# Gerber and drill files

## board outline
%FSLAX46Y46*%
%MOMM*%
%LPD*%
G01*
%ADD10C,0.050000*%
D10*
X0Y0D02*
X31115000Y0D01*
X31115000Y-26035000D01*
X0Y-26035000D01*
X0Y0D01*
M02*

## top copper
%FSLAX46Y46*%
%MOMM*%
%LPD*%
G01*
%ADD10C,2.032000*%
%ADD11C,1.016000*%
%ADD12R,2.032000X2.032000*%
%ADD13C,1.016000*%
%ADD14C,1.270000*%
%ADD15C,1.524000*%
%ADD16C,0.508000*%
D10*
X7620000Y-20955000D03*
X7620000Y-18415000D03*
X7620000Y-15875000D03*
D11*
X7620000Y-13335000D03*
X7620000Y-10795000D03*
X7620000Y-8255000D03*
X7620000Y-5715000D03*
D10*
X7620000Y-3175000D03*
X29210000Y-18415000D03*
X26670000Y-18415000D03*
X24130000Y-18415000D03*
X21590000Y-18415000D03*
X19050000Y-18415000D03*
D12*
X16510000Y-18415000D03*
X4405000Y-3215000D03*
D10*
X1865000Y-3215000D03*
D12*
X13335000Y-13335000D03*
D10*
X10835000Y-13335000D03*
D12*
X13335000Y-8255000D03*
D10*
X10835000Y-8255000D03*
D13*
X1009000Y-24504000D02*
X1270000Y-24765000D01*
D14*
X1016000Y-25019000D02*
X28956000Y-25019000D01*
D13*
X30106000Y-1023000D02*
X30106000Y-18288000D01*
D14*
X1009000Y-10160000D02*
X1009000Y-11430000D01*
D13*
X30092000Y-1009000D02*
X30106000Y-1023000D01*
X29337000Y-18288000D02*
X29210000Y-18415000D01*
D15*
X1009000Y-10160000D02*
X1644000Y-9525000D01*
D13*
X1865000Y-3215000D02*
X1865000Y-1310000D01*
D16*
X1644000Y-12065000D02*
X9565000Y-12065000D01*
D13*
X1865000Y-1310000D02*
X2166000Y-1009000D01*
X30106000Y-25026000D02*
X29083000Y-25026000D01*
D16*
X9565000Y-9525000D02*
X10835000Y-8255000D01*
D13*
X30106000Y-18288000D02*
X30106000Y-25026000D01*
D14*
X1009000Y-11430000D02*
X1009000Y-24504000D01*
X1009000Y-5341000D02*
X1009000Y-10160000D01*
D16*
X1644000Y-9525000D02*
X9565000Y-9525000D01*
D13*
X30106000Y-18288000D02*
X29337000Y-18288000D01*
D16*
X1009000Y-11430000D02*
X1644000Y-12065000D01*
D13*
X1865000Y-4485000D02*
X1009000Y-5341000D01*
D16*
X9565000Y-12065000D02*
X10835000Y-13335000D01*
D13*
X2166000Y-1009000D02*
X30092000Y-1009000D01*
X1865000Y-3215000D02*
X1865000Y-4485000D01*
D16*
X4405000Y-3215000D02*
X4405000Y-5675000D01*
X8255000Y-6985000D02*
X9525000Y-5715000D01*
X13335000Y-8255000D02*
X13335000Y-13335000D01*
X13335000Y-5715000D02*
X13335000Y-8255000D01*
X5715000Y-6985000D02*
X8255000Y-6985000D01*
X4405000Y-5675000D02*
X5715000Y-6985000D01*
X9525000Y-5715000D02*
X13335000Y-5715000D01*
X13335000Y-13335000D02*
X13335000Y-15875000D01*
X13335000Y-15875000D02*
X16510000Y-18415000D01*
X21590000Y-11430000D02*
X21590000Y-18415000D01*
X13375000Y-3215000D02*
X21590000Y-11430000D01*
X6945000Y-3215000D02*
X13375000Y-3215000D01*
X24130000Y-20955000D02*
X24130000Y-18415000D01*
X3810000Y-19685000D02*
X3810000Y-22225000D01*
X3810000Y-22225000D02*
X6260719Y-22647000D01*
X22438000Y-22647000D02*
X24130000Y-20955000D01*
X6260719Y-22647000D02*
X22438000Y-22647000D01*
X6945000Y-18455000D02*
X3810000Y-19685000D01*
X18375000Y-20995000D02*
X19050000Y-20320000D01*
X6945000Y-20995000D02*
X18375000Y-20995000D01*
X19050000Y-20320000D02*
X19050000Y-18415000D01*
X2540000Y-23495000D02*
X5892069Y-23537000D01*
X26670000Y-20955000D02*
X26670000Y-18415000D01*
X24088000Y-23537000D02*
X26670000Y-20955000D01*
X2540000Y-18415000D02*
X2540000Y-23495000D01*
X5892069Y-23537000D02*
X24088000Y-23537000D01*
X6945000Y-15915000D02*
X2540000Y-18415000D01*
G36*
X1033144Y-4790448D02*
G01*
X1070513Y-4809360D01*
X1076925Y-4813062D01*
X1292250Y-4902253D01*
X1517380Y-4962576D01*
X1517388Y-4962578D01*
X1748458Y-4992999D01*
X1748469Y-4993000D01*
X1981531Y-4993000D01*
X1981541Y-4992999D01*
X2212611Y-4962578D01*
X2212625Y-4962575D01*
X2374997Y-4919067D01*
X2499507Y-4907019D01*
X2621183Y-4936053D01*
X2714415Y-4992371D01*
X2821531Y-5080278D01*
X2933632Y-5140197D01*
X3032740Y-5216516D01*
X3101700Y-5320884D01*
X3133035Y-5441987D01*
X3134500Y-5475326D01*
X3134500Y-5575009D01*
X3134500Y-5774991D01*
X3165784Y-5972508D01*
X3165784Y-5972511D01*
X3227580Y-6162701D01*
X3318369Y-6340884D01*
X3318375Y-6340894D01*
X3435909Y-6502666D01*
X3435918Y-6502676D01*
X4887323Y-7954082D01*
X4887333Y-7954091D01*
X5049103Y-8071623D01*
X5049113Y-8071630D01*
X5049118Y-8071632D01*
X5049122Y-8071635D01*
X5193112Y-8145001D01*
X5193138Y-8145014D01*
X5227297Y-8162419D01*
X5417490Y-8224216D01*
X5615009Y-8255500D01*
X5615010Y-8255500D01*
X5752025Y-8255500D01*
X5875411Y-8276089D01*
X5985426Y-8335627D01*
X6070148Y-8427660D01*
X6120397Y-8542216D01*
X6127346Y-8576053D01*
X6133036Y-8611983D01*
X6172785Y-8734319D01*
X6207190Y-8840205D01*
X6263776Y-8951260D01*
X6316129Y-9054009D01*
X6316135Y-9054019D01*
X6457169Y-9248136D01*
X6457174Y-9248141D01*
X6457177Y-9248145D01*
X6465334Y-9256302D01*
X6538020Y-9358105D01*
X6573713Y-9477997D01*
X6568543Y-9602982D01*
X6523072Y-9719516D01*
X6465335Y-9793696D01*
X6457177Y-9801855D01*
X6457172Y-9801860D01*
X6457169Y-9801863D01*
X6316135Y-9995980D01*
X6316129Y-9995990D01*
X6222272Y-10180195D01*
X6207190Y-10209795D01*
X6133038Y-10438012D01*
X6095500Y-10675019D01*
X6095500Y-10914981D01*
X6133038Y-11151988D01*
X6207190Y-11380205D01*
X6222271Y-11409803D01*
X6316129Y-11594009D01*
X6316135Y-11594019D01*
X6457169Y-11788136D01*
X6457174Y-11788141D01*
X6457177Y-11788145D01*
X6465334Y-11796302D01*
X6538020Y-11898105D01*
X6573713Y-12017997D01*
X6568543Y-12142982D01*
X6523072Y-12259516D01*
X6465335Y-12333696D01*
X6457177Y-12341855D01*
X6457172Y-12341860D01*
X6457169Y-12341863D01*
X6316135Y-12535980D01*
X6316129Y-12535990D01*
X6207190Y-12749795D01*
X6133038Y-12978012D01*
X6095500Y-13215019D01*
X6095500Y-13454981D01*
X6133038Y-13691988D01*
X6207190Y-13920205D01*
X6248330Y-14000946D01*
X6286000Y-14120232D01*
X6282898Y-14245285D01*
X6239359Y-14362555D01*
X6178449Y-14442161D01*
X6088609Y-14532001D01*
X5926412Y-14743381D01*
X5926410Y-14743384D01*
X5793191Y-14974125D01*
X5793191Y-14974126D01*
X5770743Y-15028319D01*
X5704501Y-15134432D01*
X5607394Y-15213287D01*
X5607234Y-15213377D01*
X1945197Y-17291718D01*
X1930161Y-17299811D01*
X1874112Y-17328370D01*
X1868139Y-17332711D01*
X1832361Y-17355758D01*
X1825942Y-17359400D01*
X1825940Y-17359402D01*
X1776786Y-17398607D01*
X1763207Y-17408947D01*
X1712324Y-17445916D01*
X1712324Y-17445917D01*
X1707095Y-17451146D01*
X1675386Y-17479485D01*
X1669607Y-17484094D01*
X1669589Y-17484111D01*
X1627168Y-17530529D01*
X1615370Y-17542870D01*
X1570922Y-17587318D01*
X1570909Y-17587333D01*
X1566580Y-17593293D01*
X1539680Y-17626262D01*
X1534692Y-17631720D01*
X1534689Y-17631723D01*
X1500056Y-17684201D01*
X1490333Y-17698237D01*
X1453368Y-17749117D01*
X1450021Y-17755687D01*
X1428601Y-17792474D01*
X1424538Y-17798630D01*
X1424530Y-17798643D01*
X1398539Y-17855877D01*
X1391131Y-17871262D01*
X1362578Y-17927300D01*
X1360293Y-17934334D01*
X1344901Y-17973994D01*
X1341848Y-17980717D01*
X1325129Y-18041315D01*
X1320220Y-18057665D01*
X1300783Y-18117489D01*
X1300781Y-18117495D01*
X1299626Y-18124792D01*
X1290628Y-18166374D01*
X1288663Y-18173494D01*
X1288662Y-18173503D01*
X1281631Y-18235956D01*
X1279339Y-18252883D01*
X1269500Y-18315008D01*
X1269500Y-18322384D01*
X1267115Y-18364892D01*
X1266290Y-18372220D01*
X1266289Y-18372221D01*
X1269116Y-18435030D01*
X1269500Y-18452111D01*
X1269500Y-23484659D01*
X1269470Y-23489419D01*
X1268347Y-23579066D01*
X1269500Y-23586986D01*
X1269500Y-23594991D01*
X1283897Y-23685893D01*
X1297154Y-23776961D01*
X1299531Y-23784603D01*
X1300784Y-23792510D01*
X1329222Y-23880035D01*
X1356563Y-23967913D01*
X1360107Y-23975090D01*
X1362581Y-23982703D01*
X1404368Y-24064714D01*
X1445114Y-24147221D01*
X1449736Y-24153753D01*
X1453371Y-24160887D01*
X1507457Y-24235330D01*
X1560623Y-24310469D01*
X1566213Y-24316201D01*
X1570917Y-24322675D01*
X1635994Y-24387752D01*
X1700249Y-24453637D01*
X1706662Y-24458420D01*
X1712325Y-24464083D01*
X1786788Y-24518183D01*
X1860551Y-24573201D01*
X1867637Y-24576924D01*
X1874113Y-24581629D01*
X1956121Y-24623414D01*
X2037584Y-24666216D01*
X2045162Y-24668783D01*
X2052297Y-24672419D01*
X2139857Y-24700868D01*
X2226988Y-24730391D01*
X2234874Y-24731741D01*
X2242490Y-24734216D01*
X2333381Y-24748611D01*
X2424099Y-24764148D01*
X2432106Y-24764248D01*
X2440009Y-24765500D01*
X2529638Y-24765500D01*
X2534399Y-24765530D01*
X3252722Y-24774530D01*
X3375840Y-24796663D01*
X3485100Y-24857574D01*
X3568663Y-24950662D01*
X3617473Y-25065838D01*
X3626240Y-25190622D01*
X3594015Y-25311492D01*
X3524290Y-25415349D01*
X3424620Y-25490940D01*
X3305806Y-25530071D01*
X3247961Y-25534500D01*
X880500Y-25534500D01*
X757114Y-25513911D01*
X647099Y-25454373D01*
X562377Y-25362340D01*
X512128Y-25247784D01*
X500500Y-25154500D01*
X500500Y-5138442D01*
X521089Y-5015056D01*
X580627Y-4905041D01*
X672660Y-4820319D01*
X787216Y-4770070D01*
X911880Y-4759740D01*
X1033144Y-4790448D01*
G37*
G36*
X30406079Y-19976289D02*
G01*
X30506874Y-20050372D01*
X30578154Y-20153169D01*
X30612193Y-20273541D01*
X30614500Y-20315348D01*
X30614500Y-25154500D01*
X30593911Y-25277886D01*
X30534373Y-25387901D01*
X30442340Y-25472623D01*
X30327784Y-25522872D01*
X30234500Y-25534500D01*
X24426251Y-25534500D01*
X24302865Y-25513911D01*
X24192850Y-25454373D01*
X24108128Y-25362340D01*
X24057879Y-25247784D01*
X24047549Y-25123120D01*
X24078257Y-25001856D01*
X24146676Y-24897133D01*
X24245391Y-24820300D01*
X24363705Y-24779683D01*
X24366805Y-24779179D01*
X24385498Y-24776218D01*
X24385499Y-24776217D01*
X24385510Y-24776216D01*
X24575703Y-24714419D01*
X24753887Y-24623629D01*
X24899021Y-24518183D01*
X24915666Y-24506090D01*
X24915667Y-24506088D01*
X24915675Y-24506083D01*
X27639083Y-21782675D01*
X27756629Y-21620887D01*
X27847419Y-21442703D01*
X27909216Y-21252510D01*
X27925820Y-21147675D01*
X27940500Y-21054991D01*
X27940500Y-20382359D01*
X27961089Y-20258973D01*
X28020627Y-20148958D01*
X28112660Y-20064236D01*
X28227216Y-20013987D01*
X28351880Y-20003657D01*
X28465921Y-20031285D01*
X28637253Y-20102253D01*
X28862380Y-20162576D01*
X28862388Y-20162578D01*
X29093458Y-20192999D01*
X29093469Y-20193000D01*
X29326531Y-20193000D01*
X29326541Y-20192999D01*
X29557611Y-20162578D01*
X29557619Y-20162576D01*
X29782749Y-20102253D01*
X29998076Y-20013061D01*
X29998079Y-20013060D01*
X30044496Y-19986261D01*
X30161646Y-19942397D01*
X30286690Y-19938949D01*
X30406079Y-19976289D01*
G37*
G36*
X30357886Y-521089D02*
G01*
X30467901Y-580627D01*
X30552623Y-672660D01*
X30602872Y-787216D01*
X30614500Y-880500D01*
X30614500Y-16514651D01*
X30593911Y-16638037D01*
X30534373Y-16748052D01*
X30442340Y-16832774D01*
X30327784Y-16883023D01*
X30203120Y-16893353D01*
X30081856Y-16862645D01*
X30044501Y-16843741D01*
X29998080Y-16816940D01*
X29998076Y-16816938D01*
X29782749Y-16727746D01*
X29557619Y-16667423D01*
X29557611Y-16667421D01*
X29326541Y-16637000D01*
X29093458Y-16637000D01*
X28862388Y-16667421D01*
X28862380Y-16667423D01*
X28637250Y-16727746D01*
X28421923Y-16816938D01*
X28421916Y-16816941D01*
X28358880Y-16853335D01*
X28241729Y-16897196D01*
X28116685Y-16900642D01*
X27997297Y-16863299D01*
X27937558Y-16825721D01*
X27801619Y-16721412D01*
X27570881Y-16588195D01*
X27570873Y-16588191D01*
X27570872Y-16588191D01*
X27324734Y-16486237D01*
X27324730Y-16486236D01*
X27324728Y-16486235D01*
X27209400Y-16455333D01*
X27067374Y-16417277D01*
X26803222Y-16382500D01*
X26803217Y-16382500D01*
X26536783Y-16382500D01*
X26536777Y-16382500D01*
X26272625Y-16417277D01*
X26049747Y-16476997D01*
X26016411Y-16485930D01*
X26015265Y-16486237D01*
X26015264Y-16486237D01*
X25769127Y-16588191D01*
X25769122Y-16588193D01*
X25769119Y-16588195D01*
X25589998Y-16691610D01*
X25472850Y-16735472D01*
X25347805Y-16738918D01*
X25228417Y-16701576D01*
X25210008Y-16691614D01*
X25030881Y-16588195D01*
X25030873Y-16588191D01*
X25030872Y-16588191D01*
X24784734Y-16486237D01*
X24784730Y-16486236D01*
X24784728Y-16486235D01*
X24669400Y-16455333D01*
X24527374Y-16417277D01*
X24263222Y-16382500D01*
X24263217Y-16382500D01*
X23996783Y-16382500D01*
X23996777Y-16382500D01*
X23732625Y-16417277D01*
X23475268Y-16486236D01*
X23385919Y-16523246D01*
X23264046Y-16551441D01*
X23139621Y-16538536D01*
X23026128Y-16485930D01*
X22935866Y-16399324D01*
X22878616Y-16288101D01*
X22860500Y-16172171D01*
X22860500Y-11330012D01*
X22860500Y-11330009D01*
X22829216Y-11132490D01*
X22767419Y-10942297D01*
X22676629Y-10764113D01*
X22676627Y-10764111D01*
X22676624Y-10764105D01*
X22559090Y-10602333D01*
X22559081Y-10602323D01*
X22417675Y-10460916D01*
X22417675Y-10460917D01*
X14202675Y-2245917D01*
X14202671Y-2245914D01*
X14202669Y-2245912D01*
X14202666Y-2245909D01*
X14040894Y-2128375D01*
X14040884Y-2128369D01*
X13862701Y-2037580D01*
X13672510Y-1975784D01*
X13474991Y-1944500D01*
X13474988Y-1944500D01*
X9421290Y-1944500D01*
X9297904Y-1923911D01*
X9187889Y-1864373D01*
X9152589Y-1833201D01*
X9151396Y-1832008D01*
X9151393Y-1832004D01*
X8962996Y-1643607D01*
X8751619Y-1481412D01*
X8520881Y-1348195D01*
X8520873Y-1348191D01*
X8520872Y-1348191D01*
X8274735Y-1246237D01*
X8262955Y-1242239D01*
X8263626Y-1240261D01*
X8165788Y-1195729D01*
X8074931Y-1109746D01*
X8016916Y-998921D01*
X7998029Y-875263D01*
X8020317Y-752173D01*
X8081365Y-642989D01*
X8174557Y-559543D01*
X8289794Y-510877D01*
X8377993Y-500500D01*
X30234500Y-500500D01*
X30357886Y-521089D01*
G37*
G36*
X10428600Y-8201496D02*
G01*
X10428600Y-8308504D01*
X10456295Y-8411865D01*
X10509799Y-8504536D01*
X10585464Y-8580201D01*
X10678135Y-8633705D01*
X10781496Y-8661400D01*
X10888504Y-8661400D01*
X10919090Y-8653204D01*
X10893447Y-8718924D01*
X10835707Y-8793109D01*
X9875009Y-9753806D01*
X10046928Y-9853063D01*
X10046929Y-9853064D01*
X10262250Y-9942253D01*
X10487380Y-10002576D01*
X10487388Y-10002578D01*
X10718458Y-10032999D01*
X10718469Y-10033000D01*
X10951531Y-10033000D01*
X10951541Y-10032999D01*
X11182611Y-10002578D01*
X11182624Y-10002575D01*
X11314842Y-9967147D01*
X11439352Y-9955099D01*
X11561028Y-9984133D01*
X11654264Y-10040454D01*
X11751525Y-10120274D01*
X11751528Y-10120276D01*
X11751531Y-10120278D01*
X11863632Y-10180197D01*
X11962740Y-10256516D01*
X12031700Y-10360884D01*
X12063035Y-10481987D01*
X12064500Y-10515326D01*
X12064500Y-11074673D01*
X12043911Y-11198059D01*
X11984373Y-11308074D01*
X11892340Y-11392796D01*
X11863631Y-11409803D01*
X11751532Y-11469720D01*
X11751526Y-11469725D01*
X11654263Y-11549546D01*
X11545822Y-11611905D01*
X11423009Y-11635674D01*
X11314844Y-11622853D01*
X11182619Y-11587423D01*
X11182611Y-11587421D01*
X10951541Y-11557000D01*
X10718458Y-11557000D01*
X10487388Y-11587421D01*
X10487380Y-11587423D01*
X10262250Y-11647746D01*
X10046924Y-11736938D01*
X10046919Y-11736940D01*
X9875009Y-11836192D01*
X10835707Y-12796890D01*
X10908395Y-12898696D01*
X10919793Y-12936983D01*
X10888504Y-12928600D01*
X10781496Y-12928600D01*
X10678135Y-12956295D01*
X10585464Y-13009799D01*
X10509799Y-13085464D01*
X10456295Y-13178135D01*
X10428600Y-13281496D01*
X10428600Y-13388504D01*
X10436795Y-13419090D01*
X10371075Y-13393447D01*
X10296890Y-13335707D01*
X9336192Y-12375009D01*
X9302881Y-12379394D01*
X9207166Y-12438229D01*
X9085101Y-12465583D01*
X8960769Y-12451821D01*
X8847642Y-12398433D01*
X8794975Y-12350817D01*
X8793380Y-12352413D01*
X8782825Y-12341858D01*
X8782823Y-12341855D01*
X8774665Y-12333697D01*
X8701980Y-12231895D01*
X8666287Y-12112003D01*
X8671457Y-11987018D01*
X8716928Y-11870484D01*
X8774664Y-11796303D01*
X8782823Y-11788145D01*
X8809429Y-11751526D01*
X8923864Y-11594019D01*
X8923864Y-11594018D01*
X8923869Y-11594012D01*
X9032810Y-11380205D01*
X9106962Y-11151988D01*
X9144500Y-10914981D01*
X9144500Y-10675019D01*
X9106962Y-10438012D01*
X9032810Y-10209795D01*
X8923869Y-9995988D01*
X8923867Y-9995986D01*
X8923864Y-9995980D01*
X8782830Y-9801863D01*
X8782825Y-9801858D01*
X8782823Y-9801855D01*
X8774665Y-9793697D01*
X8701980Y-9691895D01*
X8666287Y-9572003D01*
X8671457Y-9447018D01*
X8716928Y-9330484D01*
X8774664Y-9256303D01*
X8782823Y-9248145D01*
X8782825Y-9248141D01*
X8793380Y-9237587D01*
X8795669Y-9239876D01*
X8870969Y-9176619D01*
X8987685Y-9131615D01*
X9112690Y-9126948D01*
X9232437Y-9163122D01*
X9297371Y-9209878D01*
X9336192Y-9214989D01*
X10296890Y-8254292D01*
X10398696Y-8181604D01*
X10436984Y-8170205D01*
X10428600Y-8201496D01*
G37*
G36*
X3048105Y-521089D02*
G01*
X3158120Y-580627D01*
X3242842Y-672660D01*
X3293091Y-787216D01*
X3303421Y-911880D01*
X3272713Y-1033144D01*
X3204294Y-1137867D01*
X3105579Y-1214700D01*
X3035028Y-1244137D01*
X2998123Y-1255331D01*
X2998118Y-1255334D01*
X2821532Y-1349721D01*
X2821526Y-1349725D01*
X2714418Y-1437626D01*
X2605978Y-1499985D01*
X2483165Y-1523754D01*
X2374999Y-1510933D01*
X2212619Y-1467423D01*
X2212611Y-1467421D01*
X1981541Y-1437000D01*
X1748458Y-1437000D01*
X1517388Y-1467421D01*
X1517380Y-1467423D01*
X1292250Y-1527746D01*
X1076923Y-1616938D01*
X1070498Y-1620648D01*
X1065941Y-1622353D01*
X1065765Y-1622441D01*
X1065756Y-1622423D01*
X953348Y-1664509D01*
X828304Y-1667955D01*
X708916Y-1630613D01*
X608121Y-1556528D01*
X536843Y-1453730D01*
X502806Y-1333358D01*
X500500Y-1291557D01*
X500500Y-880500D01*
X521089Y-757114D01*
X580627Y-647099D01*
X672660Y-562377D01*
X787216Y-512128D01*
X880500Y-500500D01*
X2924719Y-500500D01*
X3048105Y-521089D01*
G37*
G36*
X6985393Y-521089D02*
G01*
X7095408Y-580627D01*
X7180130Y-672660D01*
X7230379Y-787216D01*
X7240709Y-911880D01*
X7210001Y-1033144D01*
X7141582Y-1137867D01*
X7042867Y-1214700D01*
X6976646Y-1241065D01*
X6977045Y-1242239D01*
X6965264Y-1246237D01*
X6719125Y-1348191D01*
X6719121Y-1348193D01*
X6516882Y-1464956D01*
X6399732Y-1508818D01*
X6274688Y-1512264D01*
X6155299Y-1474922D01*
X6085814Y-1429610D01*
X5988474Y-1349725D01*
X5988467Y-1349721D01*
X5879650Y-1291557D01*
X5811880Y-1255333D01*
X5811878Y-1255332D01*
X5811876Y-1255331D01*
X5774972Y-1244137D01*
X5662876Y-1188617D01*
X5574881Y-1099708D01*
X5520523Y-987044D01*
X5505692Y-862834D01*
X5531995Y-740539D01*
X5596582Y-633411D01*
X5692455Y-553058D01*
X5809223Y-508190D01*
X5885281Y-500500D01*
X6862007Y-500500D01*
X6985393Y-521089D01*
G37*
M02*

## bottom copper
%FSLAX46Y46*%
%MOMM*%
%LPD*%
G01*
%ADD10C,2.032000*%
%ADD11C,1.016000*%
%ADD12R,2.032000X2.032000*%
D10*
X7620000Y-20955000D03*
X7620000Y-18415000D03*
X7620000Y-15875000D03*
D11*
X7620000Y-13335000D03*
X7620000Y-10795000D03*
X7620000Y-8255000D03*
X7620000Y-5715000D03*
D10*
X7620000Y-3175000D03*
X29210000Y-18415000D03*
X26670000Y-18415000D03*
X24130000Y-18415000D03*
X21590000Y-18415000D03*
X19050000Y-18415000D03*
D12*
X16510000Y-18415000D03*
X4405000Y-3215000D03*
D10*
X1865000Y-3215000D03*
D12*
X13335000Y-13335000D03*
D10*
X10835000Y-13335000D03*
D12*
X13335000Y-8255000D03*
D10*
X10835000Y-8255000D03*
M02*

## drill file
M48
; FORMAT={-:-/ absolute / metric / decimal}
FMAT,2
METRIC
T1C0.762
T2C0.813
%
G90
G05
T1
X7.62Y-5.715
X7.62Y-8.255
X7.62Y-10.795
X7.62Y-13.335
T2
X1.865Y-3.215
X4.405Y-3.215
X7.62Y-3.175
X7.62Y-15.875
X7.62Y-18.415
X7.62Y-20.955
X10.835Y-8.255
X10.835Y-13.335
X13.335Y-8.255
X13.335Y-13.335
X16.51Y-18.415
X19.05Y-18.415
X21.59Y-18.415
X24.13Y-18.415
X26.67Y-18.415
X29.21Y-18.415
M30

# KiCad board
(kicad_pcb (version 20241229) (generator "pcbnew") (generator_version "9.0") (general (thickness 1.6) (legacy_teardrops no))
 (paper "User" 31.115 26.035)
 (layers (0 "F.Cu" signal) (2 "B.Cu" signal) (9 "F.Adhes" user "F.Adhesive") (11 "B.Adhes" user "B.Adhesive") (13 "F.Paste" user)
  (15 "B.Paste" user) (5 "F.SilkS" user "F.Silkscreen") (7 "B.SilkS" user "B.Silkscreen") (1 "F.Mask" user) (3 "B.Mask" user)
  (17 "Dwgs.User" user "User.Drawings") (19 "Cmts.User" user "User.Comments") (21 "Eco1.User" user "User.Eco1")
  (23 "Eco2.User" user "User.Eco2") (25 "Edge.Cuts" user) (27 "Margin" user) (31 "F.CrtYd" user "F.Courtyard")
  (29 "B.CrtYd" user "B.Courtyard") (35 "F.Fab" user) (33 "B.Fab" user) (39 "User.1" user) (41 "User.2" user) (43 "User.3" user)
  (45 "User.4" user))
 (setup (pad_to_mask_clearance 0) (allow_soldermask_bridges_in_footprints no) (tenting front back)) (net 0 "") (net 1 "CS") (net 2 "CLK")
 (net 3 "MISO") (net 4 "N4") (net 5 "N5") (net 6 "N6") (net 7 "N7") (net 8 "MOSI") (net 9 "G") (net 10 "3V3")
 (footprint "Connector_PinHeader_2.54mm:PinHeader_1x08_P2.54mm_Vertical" (layer "F.Cu") (at 7.62 20.955 180)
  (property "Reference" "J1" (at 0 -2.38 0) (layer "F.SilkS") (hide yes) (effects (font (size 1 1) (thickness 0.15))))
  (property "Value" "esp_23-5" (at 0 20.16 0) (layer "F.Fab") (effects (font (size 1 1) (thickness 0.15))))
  (pad "1" thru_hole circle (at 0 0 180) (size 2.032 2.032) (drill 0.8128) (layers "*.Cu" "*.Mask") (remove_unused_layers no) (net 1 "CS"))
  (pad "2" thru_hole circle (at 0 2.54 180) (size 2.032 2.032) (drill 0.8128) (layers "*.Cu" "*.Mask") (remove_unused_layers no)
   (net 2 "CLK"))
  (pad "3" thru_hole circle (at 0 5.08 180) (size 2.032 2.032) (drill 0.8128) (layers "*.Cu" "*.Mask") (remove_unused_layers no)
   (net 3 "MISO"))
  (pad "4" thru_hole circle (at 0 7.62 180) (size 1.016 1.016) (drill 0.762) (layers "*.Cu" "*.Mask") (remove_unused_layers no) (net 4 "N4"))
  (pad "5" thru_hole circle (at 0 10.16 180) (size 1.016 1.016) (drill 0.762) (layers "*.Cu" "*.Mask") (remove_unused_layers no)
   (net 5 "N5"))
  (pad "6" thru_hole circle (at 0 12.7 180) (size 1.016 1.016) (drill 0.762) (layers "*.Cu" "*.Mask") (remove_unused_layers no) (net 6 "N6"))
  (pad "7" thru_hole circle (at 0 15.24 180) (size 1.016 1.016) (drill 0.762) (layers "*.Cu" "*.Mask") (remove_unused_layers no)
   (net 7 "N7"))
  (pad "8" thru_hole circle (at 0 17.78 180) (size 2.032 2.032) (drill 0.8128) (layers "*.Cu" "*.Mask") (remove_unused_layers no)
   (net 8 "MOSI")))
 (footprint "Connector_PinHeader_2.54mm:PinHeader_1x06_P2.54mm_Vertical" (layer "F.Cu") (at 29.21 18.415 -90)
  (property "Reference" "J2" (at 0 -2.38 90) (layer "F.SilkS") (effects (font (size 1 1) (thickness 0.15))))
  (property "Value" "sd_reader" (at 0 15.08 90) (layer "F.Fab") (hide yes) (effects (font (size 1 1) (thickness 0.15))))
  (pad "1" thru_hole circle (at 0 0 270) (size 2.032 2.032) (drill 0.8128) (layers "*.Cu" "*.Mask") (remove_unused_layers no) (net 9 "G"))
  (pad "2" thru_hole circle (at 0 2.54 270) (size 2.032 2.032) (drill 0.8128) (layers "*.Cu" "*.Mask") (remove_unused_layers no)
   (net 3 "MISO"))
  (pad "3" thru_hole circle (at 0 5.08 270) (size 2.032 2.032) (drill 0.8128) (layers "*.Cu" "*.Mask") (remove_unused_layers no)
   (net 2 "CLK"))
  (pad "4" thru_hole circle (at 0 7.62 270) (size 2.032 2.032) (drill 0.8128) (layers "*.Cu" "*.Mask") (remove_unused_layers no)
   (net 8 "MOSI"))
  (pad "5" thru_hole circle (at 0 10.16 270) (size 2.032 2.032) (drill 0.8128) (layers "*.Cu" "*.Mask") (remove_unused_layers no)
   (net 1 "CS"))
  (pad "6" thru_hole rect (at 0 12.7 270) (size 2.032 2.032) (drill 0.8128) (layers "*.Cu" "*.Mask") (remove_unused_layers no)
   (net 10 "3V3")))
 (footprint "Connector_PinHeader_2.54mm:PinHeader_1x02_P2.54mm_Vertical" (layer "F.Cu") (at 4.405 3.215 -90)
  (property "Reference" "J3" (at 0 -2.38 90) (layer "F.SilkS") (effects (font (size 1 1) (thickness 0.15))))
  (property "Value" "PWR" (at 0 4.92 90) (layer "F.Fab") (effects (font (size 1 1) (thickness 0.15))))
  (pad "1" thru_hole rect (at 0 0 270) (size 2.032 2.032) (drill 0.8128) (layers "*.Cu" "*.Mask") (remove_unused_layers no) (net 10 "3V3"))
  (pad "2" thru_hole circle (at 0 2.54 270) (size 2.032 2.032) (drill 0.8128) (layers "*.Cu" "*.Mask") (remove_unused_layers no) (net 9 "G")))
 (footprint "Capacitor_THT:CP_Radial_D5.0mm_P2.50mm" (layer "F.Cu") (at 13.335 13.335 180)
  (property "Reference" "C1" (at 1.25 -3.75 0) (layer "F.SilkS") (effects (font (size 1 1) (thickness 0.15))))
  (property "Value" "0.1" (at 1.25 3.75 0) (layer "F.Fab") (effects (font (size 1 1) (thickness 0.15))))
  (pad "1" thru_hole rect (at 0 0 180) (size 2.032 2.032) (drill 0.8128) (layers "*.Cu" "*.Mask") (remove_unused_layers no) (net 10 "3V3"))
  (pad "2" thru_hole circle (at 2.5 0 180) (size 2.032 2.032) (drill 0.8128) (layers "*.Cu" "*.Mask") (remove_unused_layers no) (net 9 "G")))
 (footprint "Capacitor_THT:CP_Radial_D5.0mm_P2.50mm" (layer "F.Cu") (at 13.335 8.255 180)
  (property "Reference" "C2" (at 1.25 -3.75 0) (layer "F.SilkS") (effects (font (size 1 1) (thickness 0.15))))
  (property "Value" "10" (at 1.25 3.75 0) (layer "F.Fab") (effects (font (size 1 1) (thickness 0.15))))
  (pad "1" thru_hole rect (at 0 0 180) (size 2.032 2.032) (drill 0.8128) (layers "*.Cu" "*.Mask") (remove_unused_layers no) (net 10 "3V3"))
  (pad "2" thru_hole circle (at 2.5 0 180) (size 2.032 2.032) (drill 0.8128) (layers "*.Cu" "*.Mask") (remove_unused_layers no) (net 9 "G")))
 (gr_rect (start 0 0) (end 31.115 26.035) (stroke (width 0.05) (type default)) (fill no) (layer "Edge.Cuts"))
 (segment (start 1.009 24.504) (end 1.27 24.765) (width 1.016) (layer "F.Cu") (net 9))
 (segment (start 1.016 25.019) (end 28.956 25.019) (width 1.27) (layer "F.Cu") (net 9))
 (segment (start 30.106 1.023) (end 30.106 18.288) (width 1.016) (layer "F.Cu") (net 9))
 (segment (start 1.009 10.16) (end 1.009 11.43) (width 1.27) (layer "F.Cu") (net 9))
 (segment (start 30.092 1.009) (end 30.106 1.023) (width 1.016) (layer "F.Cu") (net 9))
 (segment (start 29.337 18.288) (end 29.21 18.415) (width 1.016) (layer "F.Cu") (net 9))
 (segment (start 1.009 10.16) (end 1.644 9.525) (width 1.524) (layer "F.Cu") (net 9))
 (segment (start 1.865 3.215) (end 1.865 1.31) (width 1.016) (layer "F.Cu") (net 9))
 (segment (start 1.644 12.065) (end 9.565 12.065) (width 0.508) (layer "F.Cu") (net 9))
 (segment (start 1.865 1.31) (end 2.166 1.009) (width 1.016) (layer "F.Cu") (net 9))
 (segment (start 30.106 25.026) (end 29.083 25.026) (width 1.016) (layer "F.Cu") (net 9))
 (segment (start 9.565 9.525) (end 10.835 8.255) (width 0.508) (layer "F.Cu") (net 9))
 (segment (start 30.106 18.288) (end 30.106 25.026) (width 1.016) (layer "F.Cu") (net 9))
 (segment (start 1.009 11.43) (end 1.009 24.504) (width 1.27) (layer "F.Cu") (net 9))
 (segment (start 1.009 5.341) (end 1.009 10.16) (width 1.27) (layer "F.Cu") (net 9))
 (segment (start 1.644 9.525) (end 9.565 9.525) (width 0.508) (layer "F.Cu") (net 9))
 (segment (start 30.106 18.288) (end 29.337 18.288) (width 1.016) (layer "F.Cu") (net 9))
 (segment (start 1.009 11.43) (end 1.644 12.065) (width 0.508) (layer "F.Cu") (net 9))
 (segment (start 1.865 4.485) (end 1.009 5.341) (width 1.016) (layer "F.Cu") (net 9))
 (segment (start 9.565 12.065) (end 10.835 13.335) (width 0.508) (layer "F.Cu") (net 9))
 (segment (start 2.166 1.009) (end 30.092 1.009) (width 1.016) (layer "F.Cu") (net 9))
 (segment (start 1.865 3.215) (end 1.865 4.485) (width 1.016) (layer "F.Cu") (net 9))
 (segment (start 4.405 3.215) (end 4.405 5.675) (width 0.508) (layer "F.Cu") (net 10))
 (segment (start 8.255 6.985) (end 9.525 5.715) (width 0.508) (layer "F.Cu") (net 10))
 (segment (start 13.335 8.255) (end 13.335 13.335) (width 0.508) (layer "F.Cu") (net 10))
 (segment (start 13.335 5.715) (end 13.335 8.255) (width 0.508) (layer "F.Cu") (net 10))
 (segment (start 5.715 6.985) (end 8.255 6.985) (width 0.508) (layer "F.Cu") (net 10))
 (segment (start 4.405 5.675) (end 5.715 6.985) (width 0.508) (layer "F.Cu") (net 10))
 (segment (start 9.525 5.715) (end 13.335 5.715) (width 0.508) (layer "F.Cu") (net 10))
 (segment (start 13.335 13.335) (end 13.335 15.875) (width 0.508) (layer "F.Cu") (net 10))
 (segment (start 13.335 15.875) (end 16.51 18.415) (width 0.508) (layer "F.Cu") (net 10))
 (segment (start 21.59 11.43) (end 21.59 18.415) (width 0.508) (layer "F.Cu") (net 8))
 (segment (start 13.375 3.215) (end 21.59 11.43) (width 0.508) (layer "F.Cu") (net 8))
 (segment (start 6.945 3.215) (end 13.375 3.215) (width 0.508) (layer "F.Cu") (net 8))
 (segment (start 24.13 20.955) (end 24.13 18.415) (width 0.508) (layer "F.Cu") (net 2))
 (segment (start 3.81 19.685) (end 3.81 22.225) (width 0.508) (layer "F.Cu") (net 2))
 (segment (start 3.81 22.225) (end 6.260719 22.647) (width 0.508) (layer "F.Cu") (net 2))
 (segment (start 22.438 22.647) (end 24.13 20.955) (width 0.508) (layer "F.Cu") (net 2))
 (segment (start 6.260719 22.647) (end 22.438 22.647) (width 0.508) (layer "F.Cu") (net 2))
 (segment (start 6.945 18.455) (end 3.81 19.685) (width 0.508) (layer "F.Cu") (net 2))
 (segment (start 18.375 20.995) (end 19.05 20.32) (width 0.508) (layer "F.Cu") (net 1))
 (segment (start 6.945 20.995) (end 18.375 20.995) (width 0.508) (layer "F.Cu") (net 1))
 (segment (start 19.05 20.32) (end 19.05 18.415) (width 0.508) (layer "F.Cu") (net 1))
 (segment (start 2.54 23.495) (end 5.892069 23.537) (width 0.508) (layer "F.Cu") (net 3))
 (segment (start 26.67 20.955) (end 26.67 18.415) (width 0.508) (layer "F.Cu") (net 3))
 (segment (start 24.088 23.537) (end 26.67 20.955) (width 0.508) (layer "F.Cu") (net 3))
 (segment (start 2.54 18.415) (end 2.54 23.495) (width 0.508) (layer "F.Cu") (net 3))
 (segment (start 5.892069 23.537) (end 24.088 23.537) (width 0.508) (layer "F.Cu") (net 3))
 (segment (start 6.945 15.915) (end 2.54 18.415) (width 0.508) (layer "F.Cu") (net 3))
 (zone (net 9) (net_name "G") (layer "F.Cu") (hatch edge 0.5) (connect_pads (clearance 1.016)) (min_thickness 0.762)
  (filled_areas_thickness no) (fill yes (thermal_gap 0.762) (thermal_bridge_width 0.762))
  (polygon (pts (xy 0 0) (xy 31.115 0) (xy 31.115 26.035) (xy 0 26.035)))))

